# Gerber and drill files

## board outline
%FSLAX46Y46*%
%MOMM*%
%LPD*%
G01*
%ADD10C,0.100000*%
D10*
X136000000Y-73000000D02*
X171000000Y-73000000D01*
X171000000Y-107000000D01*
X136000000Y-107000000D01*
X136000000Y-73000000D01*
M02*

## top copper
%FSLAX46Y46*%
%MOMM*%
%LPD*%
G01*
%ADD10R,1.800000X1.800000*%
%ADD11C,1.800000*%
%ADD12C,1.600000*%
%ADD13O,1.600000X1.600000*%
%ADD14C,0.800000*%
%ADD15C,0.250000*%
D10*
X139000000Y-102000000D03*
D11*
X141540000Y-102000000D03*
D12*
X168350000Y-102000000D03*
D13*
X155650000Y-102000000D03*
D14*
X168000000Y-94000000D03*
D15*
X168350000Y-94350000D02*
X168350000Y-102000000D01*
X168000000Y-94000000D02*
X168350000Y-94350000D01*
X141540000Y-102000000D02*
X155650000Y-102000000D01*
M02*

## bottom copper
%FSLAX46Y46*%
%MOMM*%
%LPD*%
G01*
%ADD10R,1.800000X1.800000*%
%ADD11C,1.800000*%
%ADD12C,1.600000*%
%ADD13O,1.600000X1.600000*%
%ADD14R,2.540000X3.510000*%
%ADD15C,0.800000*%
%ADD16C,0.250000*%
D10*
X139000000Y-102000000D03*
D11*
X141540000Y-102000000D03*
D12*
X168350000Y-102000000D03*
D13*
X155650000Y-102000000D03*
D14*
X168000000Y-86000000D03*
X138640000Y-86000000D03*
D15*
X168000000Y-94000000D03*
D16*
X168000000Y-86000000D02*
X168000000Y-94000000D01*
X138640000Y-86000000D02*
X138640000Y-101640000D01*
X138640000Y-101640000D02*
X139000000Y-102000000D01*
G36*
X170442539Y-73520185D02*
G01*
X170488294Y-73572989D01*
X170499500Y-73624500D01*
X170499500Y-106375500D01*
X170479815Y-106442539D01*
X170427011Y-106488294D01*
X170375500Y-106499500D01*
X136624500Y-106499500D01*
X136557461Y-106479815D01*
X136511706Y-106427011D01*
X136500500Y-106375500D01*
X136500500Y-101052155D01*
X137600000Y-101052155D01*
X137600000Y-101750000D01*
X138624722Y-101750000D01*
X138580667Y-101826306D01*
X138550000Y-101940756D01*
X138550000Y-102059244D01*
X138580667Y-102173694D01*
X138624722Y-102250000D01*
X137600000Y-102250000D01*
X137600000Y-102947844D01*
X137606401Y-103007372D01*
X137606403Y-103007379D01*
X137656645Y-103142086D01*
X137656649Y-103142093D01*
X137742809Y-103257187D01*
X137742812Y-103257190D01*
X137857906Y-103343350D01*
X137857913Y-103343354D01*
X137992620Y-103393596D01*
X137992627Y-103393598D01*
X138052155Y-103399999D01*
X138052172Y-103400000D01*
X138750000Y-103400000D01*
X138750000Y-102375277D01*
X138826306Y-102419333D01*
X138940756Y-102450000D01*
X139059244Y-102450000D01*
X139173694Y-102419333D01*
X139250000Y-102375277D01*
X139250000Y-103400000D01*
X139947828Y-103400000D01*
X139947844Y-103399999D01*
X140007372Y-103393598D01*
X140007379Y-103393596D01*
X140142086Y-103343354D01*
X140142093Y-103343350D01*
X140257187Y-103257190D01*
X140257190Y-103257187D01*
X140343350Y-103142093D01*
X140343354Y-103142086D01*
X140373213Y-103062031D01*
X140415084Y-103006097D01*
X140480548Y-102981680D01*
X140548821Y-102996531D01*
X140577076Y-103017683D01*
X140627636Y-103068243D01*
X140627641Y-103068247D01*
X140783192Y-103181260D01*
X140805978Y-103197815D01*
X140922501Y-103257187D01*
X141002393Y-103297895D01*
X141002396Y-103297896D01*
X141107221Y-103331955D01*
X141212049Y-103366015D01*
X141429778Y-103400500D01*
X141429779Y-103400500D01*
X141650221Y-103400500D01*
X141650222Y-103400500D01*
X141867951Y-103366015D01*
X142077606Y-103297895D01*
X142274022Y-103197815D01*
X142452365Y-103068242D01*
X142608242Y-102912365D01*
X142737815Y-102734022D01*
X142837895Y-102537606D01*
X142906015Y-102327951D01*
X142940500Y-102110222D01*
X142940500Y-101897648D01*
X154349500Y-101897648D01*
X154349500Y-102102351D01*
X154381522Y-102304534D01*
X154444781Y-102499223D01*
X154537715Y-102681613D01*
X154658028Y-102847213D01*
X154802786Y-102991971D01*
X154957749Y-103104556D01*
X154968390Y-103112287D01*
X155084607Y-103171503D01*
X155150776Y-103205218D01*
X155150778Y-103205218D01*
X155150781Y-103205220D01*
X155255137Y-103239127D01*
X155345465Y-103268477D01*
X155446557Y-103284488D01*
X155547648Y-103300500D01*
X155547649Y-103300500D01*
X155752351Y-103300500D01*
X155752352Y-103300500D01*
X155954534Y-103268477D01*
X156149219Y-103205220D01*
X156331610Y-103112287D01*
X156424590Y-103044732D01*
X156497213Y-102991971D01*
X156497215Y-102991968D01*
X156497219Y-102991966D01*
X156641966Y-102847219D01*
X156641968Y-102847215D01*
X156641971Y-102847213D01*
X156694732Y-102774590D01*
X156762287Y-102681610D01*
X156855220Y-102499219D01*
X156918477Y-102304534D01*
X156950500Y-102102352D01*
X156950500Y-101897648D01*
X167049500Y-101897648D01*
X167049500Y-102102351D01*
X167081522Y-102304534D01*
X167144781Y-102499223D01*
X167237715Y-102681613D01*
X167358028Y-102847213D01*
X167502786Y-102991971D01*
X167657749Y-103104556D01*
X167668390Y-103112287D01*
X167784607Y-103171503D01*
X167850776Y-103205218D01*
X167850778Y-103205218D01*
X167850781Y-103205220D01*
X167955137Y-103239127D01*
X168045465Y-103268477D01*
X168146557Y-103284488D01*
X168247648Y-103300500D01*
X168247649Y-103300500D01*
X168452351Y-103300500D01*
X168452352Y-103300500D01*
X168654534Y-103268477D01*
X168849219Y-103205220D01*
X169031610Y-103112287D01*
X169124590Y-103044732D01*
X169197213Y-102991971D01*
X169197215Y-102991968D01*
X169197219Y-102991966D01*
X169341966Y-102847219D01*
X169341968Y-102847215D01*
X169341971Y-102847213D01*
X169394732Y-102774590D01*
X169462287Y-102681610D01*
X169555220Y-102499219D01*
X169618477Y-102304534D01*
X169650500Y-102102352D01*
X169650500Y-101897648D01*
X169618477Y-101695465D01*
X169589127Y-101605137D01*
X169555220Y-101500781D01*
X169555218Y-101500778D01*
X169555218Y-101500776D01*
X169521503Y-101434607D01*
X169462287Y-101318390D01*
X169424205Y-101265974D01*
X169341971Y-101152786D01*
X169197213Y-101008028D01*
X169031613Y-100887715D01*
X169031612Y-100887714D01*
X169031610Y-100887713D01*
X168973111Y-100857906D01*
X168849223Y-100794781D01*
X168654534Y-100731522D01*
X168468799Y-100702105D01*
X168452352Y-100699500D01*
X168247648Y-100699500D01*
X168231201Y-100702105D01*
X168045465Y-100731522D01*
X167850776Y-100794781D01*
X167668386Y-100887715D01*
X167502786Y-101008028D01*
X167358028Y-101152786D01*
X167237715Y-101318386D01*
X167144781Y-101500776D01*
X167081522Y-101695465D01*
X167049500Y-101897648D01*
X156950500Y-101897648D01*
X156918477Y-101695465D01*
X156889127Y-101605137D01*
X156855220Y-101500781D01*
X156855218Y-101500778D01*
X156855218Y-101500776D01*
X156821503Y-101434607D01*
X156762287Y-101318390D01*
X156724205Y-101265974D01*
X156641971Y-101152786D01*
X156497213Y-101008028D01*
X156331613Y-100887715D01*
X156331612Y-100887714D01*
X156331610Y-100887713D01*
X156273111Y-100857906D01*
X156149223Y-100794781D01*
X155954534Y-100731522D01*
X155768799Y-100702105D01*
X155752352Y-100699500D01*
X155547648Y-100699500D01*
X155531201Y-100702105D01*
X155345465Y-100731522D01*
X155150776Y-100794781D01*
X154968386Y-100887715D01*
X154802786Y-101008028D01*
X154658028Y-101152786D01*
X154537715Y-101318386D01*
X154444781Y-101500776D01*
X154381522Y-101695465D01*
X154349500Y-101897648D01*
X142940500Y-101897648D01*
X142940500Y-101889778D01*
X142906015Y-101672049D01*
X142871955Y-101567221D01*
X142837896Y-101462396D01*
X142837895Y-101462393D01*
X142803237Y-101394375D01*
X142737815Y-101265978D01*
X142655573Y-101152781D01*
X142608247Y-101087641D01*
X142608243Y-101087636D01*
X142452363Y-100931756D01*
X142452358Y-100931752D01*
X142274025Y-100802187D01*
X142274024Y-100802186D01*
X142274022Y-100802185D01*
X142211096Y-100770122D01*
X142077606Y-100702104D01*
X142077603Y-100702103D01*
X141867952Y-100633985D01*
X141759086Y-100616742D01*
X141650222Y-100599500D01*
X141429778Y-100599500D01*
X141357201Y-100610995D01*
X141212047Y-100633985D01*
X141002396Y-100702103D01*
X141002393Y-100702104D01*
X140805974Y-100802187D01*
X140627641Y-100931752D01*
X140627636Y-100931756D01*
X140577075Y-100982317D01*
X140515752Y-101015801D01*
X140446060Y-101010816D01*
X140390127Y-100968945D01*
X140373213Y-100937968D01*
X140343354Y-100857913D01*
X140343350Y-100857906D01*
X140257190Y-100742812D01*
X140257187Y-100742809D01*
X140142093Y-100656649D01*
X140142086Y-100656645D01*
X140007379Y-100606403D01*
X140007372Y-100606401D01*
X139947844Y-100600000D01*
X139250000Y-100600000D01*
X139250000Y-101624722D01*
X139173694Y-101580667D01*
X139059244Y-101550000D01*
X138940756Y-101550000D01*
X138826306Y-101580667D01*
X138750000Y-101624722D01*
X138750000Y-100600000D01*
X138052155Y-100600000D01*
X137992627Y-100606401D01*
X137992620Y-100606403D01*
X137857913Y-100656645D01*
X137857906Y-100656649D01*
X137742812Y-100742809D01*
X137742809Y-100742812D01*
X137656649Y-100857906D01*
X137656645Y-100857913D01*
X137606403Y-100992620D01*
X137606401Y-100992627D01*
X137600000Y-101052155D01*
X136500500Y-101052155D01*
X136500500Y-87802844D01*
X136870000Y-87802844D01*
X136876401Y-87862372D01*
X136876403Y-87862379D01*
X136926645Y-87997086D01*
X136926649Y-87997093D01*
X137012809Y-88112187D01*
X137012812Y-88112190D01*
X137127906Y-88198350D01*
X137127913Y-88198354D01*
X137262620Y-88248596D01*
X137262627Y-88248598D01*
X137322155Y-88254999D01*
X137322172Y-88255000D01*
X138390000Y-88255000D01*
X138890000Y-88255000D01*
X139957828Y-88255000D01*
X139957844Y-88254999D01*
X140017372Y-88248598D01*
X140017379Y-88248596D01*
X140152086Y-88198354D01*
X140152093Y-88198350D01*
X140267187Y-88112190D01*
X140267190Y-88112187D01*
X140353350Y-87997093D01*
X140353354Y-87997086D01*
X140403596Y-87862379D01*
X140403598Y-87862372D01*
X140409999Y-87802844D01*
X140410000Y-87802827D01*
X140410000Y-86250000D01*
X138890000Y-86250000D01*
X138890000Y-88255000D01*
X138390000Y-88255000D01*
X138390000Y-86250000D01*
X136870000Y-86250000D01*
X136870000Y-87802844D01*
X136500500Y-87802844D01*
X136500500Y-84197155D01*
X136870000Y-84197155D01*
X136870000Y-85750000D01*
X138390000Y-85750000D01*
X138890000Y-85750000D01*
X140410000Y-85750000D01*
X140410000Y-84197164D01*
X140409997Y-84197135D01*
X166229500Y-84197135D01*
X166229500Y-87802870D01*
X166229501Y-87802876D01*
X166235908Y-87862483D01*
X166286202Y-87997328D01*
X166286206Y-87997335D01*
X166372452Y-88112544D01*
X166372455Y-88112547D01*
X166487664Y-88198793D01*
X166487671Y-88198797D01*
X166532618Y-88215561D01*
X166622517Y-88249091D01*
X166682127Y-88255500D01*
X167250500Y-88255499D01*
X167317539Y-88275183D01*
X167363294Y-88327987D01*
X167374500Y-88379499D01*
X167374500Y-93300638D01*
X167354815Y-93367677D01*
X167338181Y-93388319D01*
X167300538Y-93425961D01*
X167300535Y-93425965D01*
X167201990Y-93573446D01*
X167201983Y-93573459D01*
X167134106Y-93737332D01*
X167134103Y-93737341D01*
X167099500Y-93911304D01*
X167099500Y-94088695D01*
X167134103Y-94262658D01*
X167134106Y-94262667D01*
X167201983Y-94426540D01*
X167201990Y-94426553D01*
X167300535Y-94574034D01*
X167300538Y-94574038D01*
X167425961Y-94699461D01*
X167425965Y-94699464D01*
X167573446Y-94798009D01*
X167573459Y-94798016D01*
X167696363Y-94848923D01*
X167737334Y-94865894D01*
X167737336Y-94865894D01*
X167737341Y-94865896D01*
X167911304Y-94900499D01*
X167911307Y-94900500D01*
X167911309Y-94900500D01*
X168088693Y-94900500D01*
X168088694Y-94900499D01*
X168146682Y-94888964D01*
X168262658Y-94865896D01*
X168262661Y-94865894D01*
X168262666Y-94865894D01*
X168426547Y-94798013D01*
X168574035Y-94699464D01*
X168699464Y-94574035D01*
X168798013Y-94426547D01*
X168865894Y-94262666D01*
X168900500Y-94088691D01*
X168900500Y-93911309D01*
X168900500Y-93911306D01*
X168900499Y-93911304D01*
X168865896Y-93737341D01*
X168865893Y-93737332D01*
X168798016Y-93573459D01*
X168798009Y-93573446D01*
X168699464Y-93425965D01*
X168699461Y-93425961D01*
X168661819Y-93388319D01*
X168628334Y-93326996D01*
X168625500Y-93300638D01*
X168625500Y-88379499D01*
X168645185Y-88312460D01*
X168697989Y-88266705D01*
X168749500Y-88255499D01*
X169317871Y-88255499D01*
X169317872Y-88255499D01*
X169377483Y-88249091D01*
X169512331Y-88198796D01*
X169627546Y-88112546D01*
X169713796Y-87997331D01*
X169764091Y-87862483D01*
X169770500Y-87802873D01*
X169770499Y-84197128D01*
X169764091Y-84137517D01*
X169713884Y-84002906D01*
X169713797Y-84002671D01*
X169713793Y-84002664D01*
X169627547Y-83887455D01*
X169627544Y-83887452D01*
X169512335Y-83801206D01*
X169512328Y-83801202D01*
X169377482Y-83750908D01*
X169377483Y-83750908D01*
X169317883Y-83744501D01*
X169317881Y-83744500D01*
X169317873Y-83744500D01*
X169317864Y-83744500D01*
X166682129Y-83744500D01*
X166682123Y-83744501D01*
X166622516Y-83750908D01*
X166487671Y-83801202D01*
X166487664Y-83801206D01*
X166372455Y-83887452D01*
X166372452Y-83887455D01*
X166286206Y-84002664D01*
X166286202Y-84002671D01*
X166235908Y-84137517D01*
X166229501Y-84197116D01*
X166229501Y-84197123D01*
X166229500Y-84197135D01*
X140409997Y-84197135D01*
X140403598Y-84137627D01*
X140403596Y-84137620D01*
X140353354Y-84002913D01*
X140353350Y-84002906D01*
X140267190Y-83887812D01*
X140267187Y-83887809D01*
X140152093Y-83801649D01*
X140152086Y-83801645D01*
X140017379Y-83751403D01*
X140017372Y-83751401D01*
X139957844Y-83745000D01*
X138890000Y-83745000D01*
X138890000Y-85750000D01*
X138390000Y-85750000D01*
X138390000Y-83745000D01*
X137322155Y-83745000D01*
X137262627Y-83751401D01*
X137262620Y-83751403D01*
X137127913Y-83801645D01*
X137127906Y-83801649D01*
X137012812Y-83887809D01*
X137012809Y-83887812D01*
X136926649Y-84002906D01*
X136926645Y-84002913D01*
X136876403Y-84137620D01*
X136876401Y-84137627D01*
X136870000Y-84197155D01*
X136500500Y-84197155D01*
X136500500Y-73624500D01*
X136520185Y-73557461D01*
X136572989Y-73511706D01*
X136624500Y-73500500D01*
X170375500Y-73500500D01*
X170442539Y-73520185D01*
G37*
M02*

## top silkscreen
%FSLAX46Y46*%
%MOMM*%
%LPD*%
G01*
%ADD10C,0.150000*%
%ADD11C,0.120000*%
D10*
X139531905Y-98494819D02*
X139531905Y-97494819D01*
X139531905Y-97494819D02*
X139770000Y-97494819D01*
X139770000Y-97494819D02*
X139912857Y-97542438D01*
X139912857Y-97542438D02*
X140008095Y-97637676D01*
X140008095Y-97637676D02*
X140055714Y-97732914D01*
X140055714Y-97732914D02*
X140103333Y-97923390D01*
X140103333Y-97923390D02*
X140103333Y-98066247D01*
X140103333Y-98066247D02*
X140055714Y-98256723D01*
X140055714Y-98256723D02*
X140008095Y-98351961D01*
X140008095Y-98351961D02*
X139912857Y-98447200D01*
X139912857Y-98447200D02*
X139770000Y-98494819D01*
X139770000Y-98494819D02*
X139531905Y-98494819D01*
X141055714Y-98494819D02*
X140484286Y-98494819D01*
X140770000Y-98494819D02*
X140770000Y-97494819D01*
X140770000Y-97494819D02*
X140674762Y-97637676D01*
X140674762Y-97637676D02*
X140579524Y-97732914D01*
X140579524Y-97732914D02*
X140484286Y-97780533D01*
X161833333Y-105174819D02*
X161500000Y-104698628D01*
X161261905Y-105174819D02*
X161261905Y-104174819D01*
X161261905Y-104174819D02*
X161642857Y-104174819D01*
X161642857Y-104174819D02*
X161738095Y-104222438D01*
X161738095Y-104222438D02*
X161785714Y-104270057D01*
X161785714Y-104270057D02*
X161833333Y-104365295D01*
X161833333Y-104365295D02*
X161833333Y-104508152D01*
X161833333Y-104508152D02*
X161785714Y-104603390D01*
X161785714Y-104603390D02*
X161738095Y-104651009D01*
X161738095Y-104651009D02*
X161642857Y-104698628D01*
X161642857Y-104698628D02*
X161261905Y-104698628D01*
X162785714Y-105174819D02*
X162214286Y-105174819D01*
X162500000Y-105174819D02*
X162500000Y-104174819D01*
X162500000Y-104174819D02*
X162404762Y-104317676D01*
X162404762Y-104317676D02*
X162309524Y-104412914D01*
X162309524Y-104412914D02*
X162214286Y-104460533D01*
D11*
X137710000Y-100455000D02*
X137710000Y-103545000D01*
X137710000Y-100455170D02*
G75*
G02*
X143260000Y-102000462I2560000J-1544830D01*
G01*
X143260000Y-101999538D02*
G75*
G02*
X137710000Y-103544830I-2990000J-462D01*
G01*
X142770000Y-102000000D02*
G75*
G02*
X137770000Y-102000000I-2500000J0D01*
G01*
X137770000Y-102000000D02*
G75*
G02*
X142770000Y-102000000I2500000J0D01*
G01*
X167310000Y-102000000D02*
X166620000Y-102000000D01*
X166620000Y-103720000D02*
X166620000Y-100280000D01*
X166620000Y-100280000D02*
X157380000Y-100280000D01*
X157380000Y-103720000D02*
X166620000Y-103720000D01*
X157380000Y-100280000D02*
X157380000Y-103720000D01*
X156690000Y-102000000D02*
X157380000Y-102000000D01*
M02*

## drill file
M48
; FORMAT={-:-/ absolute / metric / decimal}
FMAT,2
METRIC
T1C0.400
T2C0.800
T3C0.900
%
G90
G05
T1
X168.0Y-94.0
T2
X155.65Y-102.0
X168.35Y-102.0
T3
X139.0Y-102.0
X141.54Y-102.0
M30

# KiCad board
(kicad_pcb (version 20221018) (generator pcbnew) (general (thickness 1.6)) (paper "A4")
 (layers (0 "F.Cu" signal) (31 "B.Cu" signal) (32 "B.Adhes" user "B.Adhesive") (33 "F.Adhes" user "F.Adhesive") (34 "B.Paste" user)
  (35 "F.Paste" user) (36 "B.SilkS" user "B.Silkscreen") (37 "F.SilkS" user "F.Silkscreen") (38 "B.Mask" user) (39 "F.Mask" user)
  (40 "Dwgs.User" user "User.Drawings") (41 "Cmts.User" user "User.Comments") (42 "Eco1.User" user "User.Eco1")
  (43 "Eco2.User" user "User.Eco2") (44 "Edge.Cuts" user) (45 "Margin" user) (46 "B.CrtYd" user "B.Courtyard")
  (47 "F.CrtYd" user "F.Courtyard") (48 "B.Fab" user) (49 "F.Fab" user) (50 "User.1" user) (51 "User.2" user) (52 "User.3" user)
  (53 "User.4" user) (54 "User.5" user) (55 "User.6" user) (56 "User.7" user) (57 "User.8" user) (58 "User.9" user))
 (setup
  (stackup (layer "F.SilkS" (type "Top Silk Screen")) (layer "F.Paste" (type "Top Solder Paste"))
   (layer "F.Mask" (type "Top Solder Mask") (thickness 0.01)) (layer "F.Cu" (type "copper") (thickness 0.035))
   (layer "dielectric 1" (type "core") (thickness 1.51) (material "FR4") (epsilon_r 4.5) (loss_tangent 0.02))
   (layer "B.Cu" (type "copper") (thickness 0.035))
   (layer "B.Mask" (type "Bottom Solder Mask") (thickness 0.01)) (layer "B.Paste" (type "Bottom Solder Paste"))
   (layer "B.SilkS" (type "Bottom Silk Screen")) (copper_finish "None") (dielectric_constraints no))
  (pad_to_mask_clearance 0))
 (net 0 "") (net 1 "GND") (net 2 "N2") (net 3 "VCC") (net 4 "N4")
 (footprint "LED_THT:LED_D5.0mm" (layer "F.Cu") (at 139 102)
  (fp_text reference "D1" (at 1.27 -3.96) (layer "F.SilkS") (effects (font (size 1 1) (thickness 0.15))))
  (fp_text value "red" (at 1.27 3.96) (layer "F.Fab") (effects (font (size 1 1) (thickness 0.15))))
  (fp_line (start -1.29 -1.545) (end -1.29 1.545) (stroke (width 0.12) (type solid)) (layer "F.SilkS"))
  (fp_arc (start -1.29 -1.54483) (mid 2.072002 -2.880433) (end 4.26 0.000462) (stroke (width 0.12) (type solid)) (layer "F.SilkS"))
  (fp_arc (start 4.26 -0.000462) (mid 2.072002 2.880433) (end -1.29 1.54483) (stroke (width 0.12) (type solid)) (layer "F.SilkS"))
  (fp_circle (center 1.27 0) (end 3.77 0) (stroke (width 0.12) (type solid)) (fill none) (layer "F.SilkS"))
  (pad "1" thru_hole rect (at 0 0) (size 1.8 1.8) (drill 0.9) (layers "*.Cu" "*.Mask") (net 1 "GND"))
  (pad "2" thru_hole circle (at 2.54 0) (size 1.8 1.8) (drill 0.9) (layers "*.Cu" "*.Mask") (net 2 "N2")))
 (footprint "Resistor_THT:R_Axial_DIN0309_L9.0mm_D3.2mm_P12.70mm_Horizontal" (layer "F.Cu") (at 168.35 102 180)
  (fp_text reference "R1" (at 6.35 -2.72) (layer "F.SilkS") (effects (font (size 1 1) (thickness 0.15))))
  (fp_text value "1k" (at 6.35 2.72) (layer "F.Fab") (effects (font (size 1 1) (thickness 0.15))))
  (fp_line (start 1.04 0) (end 1.73 0) (stroke (width 0.12) (type solid)) (layer "F.SilkS"))
  (fp_line (start 1.73 -1.72) (end 1.73 1.72) (stroke (width 0.12) (type solid)) (layer "F.SilkS"))
  (fp_line (start 1.73 1.72) (end 10.97 1.72) (stroke (width 0.12) (type solid)) (layer "F.SilkS"))
  (fp_line (start 10.97 -1.72) (end 1.73 -1.72) (stroke (width 0.12) (type solid)) (layer "F.SilkS"))
  (fp_line (start 10.97 1.72) (end 10.97 -1.72) (stroke (width 0.12) (type solid)) (layer "F.SilkS"))
  (fp_line (start 11.66 0) (end 10.97 0) (stroke (width 0.12) (type solid)) (layer "F.SilkS"))
  (pad "1" thru_hole circle (at 0 0 180) (size 1.6 1.6) (drill 0.8) (layers "*.Cu" "*.Mask") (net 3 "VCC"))
  (pad "2" thru_hole oval (at 12.7 0 180) (size 1.6 1.6) (drill 0.8) (layers "*.Cu" "*.Mask") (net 2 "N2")))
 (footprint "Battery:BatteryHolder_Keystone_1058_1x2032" (layer "B.Cu") (at 153.32 86 180)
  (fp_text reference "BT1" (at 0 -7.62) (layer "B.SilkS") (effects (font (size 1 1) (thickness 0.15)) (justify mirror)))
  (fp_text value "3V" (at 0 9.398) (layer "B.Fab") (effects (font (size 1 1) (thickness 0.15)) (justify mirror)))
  (pad "1" smd rect (at -14.68 0 180) (size 2.54 3.51) (layers "B.Cu" "B.Paste" "B.Mask") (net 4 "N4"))
  (pad "2" smd rect (at 14.68 0 180) (size 2.54 3.51) (layers "B.Cu" "B.Paste" "B.Mask") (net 1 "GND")))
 (gr_rect (start 136 73) (end 171 107) (stroke (width 0.1) (type default)) (fill none) (layer "Edge.Cuts"))
 (segment (start 168.35 94.35) (end 168.35 102) (width 0.25) (layer "F.Cu") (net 3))
 (segment (start 168 94) (end 168.35 94.35) (width 0.25) (layer "F.Cu") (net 3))
 (via (at 168 94) (size 0.8) (drill 0.4) (layers "F.Cu" "B.Cu") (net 3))
 (segment (start 168 86) (end 168 94) (width 0.25) (layer "B.Cu") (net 3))
 (segment (start 138.64 86) (end 138.64 101.64) (width 0.25) (layer "B.Cu") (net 1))
 (segment (start 138.64 101.64) (end 139 102) (width 0.25) (layer "B.Cu") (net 1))
 (segment (start 141.54 102) (end 155.65 102) (width 0.25) (layer "F.Cu") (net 2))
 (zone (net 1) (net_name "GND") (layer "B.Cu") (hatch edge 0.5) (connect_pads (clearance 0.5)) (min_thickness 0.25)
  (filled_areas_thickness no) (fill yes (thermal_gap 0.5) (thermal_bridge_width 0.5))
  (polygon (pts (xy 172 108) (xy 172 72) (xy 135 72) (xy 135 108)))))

